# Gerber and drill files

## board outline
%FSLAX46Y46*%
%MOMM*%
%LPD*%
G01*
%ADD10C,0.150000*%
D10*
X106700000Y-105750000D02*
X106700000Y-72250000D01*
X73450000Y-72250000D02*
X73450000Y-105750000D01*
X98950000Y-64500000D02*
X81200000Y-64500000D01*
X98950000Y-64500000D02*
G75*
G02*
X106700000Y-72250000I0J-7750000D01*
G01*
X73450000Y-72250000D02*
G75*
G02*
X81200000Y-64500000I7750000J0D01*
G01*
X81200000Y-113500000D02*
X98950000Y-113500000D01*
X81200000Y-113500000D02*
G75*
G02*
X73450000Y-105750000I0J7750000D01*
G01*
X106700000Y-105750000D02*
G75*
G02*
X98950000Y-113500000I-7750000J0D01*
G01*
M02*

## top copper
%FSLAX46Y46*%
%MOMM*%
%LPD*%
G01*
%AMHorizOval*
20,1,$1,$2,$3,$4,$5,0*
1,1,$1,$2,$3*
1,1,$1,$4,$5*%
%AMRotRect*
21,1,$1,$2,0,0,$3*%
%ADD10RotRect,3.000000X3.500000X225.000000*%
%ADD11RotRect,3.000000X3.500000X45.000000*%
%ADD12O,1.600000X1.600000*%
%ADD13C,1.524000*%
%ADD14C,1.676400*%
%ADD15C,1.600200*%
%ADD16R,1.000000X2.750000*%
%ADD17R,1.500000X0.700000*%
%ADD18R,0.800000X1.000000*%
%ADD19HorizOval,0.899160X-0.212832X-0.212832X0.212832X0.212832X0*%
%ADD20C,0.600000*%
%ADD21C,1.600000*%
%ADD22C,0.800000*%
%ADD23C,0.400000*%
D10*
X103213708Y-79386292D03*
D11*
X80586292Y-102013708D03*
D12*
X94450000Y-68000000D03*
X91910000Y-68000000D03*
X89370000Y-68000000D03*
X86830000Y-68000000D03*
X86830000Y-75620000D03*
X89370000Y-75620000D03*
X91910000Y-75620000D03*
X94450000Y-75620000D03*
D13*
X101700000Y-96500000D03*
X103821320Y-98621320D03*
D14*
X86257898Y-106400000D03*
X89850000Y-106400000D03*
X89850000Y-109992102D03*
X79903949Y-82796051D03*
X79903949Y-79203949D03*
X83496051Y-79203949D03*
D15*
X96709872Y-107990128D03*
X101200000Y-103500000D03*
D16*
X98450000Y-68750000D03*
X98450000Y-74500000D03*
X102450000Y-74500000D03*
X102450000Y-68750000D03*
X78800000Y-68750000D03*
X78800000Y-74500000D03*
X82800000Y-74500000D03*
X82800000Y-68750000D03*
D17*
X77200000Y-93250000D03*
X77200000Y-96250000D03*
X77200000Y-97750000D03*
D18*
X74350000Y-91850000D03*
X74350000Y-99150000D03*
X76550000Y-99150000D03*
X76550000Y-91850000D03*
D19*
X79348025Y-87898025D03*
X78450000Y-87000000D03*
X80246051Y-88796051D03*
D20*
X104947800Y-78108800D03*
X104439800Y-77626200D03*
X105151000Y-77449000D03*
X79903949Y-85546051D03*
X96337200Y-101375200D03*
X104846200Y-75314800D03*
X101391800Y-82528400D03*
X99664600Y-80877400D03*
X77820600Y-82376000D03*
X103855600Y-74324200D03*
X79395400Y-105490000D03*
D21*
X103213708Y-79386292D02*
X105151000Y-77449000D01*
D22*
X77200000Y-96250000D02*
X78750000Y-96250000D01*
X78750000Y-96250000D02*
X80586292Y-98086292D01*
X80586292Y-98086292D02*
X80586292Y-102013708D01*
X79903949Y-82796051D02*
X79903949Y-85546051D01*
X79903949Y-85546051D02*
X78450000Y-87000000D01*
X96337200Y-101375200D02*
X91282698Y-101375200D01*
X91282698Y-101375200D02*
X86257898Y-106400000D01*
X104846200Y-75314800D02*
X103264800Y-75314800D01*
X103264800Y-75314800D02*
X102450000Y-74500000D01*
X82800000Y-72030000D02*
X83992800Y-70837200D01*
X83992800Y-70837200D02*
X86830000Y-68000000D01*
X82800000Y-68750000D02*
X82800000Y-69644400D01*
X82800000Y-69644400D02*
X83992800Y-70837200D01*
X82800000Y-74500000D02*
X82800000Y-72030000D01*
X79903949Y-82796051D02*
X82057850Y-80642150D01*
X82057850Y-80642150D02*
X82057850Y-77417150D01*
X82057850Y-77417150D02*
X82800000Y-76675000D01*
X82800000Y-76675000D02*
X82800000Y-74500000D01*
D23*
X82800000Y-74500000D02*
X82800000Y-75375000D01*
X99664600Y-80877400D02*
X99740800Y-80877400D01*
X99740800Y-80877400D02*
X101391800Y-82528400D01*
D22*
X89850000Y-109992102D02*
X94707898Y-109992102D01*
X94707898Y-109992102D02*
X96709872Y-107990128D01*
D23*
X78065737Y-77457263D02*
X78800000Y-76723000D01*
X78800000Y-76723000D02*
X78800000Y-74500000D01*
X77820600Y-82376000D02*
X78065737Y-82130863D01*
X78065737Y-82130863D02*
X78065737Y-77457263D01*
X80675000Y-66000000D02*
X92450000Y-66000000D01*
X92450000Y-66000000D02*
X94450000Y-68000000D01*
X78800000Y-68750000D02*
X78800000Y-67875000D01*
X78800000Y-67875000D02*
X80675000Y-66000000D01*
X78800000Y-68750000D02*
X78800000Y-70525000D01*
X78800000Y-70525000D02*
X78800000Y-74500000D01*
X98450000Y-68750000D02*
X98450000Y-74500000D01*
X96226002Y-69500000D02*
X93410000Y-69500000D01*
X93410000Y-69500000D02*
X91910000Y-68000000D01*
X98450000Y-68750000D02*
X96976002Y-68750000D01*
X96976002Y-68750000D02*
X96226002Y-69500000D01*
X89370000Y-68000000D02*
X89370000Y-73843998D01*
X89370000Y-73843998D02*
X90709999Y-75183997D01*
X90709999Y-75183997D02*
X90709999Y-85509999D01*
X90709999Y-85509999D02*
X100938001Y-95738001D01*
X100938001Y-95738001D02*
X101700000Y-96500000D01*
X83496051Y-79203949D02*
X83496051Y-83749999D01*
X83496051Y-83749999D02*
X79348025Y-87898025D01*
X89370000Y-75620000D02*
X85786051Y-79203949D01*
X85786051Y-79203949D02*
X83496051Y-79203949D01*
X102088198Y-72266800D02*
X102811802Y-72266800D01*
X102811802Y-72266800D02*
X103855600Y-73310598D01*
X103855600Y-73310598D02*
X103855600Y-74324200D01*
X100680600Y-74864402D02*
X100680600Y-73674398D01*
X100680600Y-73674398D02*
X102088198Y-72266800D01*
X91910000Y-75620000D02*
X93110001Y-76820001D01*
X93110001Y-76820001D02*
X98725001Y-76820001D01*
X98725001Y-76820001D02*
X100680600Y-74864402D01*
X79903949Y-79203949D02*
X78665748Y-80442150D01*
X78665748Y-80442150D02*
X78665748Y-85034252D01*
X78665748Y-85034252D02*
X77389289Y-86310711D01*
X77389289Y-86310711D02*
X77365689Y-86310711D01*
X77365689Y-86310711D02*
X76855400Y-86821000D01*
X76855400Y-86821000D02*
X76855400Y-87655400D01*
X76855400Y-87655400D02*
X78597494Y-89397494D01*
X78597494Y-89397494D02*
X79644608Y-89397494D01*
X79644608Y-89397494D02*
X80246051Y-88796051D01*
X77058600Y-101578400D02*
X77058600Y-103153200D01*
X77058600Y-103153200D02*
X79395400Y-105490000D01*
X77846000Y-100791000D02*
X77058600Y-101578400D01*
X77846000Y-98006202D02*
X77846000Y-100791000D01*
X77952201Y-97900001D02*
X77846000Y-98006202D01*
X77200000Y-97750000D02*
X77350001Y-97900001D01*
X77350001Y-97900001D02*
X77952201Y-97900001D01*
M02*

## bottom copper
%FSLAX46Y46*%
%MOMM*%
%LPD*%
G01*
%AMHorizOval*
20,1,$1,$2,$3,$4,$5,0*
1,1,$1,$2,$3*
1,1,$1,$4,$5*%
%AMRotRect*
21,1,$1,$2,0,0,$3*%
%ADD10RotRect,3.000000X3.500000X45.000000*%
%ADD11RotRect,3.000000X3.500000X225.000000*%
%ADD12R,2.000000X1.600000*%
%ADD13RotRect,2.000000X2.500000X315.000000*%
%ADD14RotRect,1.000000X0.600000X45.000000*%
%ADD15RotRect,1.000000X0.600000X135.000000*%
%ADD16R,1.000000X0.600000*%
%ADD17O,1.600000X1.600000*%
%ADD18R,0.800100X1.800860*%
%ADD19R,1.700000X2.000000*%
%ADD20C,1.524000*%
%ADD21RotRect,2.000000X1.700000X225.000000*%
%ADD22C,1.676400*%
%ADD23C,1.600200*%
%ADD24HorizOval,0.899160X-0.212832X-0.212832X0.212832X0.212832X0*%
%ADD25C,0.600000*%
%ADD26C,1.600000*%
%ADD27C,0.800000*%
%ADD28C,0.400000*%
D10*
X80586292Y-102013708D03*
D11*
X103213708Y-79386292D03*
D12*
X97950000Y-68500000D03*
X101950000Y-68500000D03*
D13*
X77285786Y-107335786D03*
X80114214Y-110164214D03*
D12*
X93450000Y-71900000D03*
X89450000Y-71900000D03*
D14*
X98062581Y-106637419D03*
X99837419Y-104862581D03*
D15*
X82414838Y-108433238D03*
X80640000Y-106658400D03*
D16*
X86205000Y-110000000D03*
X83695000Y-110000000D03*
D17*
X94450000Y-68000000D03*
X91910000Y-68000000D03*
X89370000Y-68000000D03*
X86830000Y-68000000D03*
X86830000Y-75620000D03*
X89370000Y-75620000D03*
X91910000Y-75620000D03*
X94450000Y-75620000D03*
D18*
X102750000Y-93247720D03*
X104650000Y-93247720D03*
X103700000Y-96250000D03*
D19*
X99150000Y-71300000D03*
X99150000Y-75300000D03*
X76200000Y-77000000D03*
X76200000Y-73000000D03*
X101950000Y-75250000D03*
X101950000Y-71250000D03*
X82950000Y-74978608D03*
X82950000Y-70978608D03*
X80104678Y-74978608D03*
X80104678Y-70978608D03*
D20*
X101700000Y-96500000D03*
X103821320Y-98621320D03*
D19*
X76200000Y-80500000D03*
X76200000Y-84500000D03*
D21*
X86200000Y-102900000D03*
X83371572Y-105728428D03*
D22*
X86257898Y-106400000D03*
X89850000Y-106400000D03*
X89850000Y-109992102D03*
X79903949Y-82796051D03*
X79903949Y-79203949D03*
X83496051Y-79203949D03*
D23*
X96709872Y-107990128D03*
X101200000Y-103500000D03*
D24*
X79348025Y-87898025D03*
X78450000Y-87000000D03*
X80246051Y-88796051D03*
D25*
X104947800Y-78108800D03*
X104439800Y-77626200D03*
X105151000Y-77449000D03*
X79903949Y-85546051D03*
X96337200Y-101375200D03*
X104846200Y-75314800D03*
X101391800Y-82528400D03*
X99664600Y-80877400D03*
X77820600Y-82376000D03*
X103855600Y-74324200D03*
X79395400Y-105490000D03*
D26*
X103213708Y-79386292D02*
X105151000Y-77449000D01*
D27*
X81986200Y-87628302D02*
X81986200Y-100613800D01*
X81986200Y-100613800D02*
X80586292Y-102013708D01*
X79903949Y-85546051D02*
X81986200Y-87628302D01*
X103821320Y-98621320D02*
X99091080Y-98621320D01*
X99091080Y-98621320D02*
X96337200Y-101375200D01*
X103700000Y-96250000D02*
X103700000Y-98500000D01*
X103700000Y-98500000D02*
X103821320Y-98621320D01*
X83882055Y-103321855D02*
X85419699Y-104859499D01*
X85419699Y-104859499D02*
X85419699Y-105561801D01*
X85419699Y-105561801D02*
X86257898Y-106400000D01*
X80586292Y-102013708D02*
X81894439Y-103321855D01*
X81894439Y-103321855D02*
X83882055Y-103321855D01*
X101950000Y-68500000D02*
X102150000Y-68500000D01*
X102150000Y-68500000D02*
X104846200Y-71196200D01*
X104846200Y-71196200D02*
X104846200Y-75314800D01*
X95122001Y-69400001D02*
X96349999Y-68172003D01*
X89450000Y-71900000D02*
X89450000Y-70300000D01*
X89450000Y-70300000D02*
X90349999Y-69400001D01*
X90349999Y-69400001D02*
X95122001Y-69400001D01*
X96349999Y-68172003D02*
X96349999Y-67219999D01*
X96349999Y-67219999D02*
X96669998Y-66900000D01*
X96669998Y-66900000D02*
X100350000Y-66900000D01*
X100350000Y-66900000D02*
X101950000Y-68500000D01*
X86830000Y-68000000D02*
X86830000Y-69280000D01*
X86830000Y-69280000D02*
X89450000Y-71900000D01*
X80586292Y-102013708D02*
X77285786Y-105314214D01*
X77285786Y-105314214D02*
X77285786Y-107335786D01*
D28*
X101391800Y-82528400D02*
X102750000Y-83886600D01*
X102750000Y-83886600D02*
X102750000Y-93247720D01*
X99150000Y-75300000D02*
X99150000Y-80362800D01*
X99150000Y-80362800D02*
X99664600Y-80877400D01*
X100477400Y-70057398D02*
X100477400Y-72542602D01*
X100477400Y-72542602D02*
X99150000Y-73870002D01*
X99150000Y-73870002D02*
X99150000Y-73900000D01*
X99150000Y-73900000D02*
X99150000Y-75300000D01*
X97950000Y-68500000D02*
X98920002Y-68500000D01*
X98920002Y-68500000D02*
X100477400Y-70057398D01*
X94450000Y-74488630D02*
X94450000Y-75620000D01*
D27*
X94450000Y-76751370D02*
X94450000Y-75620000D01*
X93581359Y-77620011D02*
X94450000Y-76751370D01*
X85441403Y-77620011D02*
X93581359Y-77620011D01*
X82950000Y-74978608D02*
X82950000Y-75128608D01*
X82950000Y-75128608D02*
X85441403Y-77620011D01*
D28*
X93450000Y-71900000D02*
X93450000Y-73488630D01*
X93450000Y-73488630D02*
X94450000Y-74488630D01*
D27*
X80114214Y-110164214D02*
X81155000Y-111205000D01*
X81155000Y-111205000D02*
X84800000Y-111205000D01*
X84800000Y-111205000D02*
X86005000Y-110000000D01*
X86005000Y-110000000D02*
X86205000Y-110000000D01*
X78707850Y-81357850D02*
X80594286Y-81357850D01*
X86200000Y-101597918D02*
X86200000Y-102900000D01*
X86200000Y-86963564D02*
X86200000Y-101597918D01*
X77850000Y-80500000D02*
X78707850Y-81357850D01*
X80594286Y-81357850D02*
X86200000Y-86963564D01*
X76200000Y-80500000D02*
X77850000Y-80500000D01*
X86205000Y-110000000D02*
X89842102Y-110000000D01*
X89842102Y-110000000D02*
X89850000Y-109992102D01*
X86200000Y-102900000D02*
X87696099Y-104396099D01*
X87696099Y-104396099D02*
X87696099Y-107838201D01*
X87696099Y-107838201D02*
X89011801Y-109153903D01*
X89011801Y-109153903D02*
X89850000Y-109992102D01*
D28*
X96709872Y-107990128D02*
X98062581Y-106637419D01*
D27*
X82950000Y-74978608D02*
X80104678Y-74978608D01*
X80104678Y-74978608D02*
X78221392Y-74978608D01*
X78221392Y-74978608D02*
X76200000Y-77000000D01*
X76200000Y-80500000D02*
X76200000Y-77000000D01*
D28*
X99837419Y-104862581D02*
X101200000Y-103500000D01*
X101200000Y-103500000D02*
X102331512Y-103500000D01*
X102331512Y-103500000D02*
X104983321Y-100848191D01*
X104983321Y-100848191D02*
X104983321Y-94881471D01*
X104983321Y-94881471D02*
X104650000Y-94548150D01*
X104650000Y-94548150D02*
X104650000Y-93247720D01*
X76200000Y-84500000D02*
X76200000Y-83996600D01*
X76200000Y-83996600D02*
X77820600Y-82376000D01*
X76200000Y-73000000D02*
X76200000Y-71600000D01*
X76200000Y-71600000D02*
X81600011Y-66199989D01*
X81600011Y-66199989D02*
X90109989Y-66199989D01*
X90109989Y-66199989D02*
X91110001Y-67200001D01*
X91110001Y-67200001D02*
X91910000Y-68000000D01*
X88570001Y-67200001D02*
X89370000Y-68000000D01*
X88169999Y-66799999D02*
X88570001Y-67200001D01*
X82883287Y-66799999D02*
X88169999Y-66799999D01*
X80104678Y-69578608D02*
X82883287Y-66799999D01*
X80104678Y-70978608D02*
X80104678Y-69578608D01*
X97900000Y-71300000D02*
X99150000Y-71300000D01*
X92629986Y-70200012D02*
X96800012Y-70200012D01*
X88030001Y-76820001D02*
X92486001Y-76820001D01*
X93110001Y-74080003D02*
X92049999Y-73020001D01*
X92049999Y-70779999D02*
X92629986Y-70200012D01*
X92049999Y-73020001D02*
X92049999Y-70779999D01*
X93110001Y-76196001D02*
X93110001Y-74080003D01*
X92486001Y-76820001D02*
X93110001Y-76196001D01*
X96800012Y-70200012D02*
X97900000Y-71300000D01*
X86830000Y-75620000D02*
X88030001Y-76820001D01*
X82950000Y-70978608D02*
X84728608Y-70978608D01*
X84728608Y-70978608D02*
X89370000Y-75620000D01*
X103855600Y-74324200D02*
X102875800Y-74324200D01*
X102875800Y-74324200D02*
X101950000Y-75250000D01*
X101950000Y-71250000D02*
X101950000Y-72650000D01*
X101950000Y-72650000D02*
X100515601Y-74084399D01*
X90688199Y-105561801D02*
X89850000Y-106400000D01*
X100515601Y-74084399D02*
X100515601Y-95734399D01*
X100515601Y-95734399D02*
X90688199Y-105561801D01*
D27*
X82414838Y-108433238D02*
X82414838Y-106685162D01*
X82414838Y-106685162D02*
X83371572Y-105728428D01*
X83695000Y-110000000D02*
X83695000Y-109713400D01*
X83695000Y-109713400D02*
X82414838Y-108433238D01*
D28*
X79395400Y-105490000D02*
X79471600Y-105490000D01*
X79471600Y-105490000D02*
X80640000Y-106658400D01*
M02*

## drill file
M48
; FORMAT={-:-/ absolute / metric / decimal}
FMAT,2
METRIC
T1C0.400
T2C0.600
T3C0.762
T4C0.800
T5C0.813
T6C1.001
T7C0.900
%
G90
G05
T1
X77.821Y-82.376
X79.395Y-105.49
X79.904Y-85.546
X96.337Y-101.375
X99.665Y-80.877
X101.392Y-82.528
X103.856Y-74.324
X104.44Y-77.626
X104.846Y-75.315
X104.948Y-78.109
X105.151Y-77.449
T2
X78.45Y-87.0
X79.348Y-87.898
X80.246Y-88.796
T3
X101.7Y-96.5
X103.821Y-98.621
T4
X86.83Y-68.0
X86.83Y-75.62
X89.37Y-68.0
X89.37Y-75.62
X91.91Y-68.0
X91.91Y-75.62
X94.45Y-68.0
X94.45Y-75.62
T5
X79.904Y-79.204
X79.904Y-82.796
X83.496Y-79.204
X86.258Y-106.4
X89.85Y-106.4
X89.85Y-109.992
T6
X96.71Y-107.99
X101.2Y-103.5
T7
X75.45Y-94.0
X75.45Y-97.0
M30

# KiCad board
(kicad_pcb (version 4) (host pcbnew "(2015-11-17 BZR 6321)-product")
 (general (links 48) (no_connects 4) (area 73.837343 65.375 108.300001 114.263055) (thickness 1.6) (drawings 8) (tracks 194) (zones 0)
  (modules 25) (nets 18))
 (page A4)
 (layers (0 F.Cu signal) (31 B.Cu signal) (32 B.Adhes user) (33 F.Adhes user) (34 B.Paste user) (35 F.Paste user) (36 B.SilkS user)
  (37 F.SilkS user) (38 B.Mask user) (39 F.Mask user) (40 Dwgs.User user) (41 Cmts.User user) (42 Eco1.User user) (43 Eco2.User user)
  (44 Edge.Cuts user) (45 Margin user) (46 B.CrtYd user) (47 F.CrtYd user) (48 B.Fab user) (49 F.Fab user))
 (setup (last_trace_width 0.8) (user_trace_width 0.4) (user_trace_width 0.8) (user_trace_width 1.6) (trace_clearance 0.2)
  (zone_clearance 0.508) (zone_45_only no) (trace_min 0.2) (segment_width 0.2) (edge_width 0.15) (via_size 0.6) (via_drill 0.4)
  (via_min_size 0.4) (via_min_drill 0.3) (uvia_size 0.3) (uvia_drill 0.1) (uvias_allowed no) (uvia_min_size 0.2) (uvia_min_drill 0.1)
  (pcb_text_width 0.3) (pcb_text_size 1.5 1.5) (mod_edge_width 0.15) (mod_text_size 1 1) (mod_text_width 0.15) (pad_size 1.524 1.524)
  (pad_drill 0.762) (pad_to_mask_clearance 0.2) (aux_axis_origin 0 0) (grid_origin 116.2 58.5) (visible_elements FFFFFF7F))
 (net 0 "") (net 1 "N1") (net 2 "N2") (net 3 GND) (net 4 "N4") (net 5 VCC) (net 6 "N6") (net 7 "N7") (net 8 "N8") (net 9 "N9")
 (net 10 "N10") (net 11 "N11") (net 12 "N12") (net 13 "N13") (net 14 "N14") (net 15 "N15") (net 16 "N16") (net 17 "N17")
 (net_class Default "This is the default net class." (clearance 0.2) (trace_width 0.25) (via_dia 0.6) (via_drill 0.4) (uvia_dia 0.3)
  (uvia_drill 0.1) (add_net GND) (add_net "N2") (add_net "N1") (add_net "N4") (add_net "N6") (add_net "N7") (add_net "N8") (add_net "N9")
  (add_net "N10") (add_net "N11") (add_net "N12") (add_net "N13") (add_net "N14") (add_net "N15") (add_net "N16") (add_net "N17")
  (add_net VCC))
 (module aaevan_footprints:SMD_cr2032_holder (layer F.Cu) (at 91.9 90.7 225)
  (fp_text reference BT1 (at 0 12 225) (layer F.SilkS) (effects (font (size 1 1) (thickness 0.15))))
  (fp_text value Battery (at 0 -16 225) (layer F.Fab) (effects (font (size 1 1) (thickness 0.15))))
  (pad 2 smd rect (at -16 0 225) (size 3 3.5) (layers F.Cu F.Paste F.Mask) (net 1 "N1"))
  (pad 1 smd rect (at 16 0 45) (size 3 3.5) (layers F.Cu F.Paste F.Mask) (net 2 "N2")))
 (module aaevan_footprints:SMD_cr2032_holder (layer B.Cu) (at 91.9 90.7 45)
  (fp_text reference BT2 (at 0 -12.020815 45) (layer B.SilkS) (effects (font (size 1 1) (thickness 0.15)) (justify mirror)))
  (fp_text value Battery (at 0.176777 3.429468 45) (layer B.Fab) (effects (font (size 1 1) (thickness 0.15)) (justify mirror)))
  (pad 2 smd rect (at -16 0 45) (size 3 3.5) (layers B.Cu B.Paste B.Mask) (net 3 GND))
  (pad 1 smd rect (at 16 0 225) (size 3 3.5) (layers B.Cu B.Paste B.Mask) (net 1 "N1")))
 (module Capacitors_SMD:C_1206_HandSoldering (layer B.Cu) (at 99.95 68.5)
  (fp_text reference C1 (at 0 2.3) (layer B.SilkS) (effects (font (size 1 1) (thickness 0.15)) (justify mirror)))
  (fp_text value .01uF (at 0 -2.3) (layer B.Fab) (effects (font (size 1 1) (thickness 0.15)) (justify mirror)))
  (pad 1 smd rect (at -2 0) (size 2 1.6) (layers B.Cu B.Paste B.Mask) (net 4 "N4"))
  (pad 2 smd rect (at 2 0) (size 2 1.6) (layers B.Cu B.Paste B.Mask) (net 3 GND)))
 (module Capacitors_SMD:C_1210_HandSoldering (layer B.Cu) (at 78.7 108.75 315)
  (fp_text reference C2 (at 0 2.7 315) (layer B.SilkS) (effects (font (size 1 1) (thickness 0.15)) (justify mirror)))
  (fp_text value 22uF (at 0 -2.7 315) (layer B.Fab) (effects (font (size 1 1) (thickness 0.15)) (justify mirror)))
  (pad 1 smd rect (at -2 0 315) (size 2 2.5) (layers B.Cu B.Paste B.Mask) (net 3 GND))
  (pad 2 smd rect (at 2 0 315) (size 2 2.5) (layers B.Cu B.Paste B.Mask) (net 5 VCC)))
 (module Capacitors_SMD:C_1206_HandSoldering (layer B.Cu) (at 91.45 71.9 180)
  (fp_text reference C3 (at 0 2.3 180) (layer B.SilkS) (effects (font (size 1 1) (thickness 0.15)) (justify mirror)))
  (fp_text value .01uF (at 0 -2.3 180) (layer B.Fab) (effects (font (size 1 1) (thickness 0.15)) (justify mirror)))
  (pad 1 smd rect (at -2 0 180) (size 2 1.6) (layers B.Cu B.Paste B.Mask) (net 5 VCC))
  (pad 2 smd rect (at 2 0 180) (size 2 1.6) (layers B.Cu B.Paste B.Mask) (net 3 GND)))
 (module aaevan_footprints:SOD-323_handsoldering (layer B.Cu) (at 98.95 105.75 45)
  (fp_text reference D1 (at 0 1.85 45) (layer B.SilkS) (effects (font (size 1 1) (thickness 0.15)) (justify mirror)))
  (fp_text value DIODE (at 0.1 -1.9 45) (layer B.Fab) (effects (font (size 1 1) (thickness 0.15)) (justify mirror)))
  (pad 1 smd rect (at -1.255 0 45) (size 1 0.6) (layers B.Cu B.Paste B.Mask) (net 5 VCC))
  (pad 2 smd rect (at 1.255 0 45) (size 1 0.6) (layers B.Cu B.Paste B.Mask) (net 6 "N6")))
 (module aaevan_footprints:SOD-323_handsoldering (layer B.Cu) (at 81.527419 107.545819 135)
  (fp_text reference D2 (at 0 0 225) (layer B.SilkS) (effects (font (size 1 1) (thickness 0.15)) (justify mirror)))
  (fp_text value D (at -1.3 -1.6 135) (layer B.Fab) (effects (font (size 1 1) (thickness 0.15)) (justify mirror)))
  (pad 1 smd rect (at -1.255 0 135) (size 1 0.6) (layers B.Cu B.Paste B.Mask) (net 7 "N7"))
  (pad 2 smd rect (at 1.255 0 135) (size 1 0.6) (layers B.Cu B.Paste B.Mask) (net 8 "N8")))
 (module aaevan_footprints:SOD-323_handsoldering (layer B.Cu) (at 84.95 110 180)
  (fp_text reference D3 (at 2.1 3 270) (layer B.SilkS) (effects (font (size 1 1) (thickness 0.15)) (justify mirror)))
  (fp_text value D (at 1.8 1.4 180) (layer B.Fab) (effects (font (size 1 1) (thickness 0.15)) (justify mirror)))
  (pad 1 smd rect (at -1.255 0 180) (size 1 0.6) (layers B.Cu B.Paste B.Mask) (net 5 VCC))
  (pad 2 smd rect (at 1.255 0 180) (size 1 0.6) (layers B.Cu B.Paste B.Mask) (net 7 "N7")))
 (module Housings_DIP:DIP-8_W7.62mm (layer F.Cu) (at 94.45 68 270)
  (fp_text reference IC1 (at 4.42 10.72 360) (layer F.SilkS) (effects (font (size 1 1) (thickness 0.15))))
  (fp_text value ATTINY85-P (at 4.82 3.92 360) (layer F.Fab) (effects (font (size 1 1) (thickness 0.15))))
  (pad 1 thru_hole oval (at 0 0 270) (size 1.6 1.6) (drill 0.8) (layers *.Cu *.Mask F.SilkS) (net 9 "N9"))
  (pad 2 thru_hole oval (at 0 2.54 270) (size 1.6 1.6) (drill 0.8) (layers *.Cu *.Mask F.SilkS) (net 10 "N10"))
  (pad 3 thru_hole oval (at 0 5.08 270) (size 1.6 1.6) (drill 0.8) (layers *.Cu *.Mask F.SilkS) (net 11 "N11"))
  (pad 4 thru_hole oval (at 0 7.62 270) (size 1.6 1.6) (drill 0.8) (layers *.Cu *.Mask F.SilkS) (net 3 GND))
  (pad 5 thru_hole oval (at 7.62 7.62 270) (size 1.6 1.6) (drill 0.8) (layers *.Cu *.Mask F.SilkS) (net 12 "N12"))
  (pad 6 thru_hole oval (at 7.62 5.08 270) (size 1.6 1.6) (drill 0.8) (layers *.Cu *.Mask F.SilkS) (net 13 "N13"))
  (pad 7 thru_hole oval (at 7.62 2.54 270) (size 1.6 1.6) (drill 0.8) (layers *.Cu *.Mask F.SilkS) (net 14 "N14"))
  (pad 8 thru_hole oval (at 7.62 0 270) (size 1.6 1.6) (drill 0.8) (layers *.Cu *.Mask F.SilkS) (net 5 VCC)))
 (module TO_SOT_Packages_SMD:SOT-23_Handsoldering (layer B.Cu) (at 103.7 94.74886)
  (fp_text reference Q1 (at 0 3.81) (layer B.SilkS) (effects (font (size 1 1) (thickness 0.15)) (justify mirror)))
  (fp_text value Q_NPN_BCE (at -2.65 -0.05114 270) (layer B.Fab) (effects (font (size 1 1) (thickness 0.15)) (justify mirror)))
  (pad 1 smd rect (at -0.95 -1.50114) (size 0.8001 1.80086) (layers B.Cu B.Paste B.Mask) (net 4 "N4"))
  (pad 2 smd rect (at 0.95 -1.50114) (size 0.8001 1.80086) (layers B.Cu B.Paste B.Mask) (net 6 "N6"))
  (pad 3 smd rect (at 0 1.50114) (size 0.8001 1.80086) (layers B.Cu B.Paste B.Mask) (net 3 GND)))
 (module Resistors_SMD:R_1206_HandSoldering (layer B.Cu) (at 99.15 73.3 270)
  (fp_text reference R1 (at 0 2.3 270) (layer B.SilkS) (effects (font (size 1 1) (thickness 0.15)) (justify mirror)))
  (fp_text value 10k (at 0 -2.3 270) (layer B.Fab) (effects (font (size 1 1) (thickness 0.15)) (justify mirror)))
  (pad 1 smd rect (at -2 0 270) (size 2 1.7) (layers B.Cu B.Paste B.Mask) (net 12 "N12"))
  (pad 2 smd rect (at 2 0 270) (size 2 1.7) (layers B.Cu B.Paste B.Mask) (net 4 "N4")))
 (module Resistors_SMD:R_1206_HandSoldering (layer B.Cu) (at 76.2 75 90)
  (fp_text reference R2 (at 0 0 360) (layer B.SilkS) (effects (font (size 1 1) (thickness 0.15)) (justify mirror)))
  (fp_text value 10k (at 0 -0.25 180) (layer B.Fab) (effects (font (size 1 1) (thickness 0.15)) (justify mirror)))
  (pad 1 smd rect (at -2 0 90) (size 2 1.7) (layers B.Cu B.Paste B.Mask) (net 5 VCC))
  (pad 2 smd rect (at 2 0 90) (size 2 1.7) (layers B.Cu B.Paste B.Mask) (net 10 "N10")))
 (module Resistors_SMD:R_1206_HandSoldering (layer B.Cu) (at 101.95 73.25 90)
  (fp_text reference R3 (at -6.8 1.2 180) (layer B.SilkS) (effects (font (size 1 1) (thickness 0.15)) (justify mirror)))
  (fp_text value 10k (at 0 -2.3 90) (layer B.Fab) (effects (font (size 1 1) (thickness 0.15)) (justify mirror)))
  (pad 1 smd rect (at -2 0 90) (size 2 1.7) (layers B.Cu B.Paste B.Mask) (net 14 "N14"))
  (pad 2 smd rect (at 2 0 90) (size 2 1.7) (layers B.Cu B.Paste B.Mask) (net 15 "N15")))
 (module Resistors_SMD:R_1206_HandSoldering (layer B.Cu) (at 82.95 72.978608 90)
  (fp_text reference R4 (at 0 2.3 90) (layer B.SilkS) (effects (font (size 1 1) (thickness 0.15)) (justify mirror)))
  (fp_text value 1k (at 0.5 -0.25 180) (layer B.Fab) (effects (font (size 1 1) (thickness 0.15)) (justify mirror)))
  (pad 1 smd rect (at -2 0 90) (size 2 1.7) (layers B.Cu B.Paste B.Mask) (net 5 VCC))
  (pad 2 smd rect (at 2 0 90) (size 2 1.7) (layers B.Cu B.Paste B.Mask) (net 13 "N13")))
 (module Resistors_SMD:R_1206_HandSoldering (layer B.Cu) (at 80.104678 72.978608 90)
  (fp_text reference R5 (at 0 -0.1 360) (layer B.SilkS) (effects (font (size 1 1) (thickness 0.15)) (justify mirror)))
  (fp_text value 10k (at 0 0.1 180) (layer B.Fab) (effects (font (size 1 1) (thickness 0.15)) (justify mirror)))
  (pad 1 smd rect (at -2 0 90) (size 2 1.7) (layers B.Cu B.Paste B.Mask) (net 5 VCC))
  (pad 2 smd rect (at 2 0 90) (size 2 1.7) (layers B.Cu B.Paste B.Mask) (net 11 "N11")))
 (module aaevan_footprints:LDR (layer F.Cu) (at 102.76066 97.56066 315)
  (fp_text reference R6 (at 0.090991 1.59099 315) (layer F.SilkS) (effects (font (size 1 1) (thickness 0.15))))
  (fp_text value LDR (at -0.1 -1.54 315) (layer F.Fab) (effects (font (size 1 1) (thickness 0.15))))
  (pad 1 thru_hole circle (at -1.5 0 315) (size 1.524 1.524) (drill 0.762) (layers *.Cu *.Mask F.SilkS) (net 11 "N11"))
  (pad 2 thru_hole circle (at 1.5 0 315) (size 1.524 1.524) (drill 0.762) (layers *.Cu *.Mask F.SilkS) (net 3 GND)))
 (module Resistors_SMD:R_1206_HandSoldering (layer B.Cu) (at 76.2 82.5 270)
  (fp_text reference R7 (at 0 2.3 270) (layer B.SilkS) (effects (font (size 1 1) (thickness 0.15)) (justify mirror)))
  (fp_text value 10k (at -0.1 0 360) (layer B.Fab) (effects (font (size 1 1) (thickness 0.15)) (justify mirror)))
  (pad 1 smd rect (at -2 0 270) (size 2 1.7) (layers B.Cu B.Paste B.Mask) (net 5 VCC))
  (pad 2 smd rect (at 2 0 270) (size 2 1.7) (layers B.Cu B.Paste B.Mask) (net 9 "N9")))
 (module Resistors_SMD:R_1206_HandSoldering (layer B.Cu) (at 84.785786 104.314214 225)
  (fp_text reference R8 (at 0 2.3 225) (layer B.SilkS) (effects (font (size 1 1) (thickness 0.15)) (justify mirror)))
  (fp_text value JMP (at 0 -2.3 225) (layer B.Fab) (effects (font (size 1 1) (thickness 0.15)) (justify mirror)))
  (pad 1 smd rect (at -2 0 225) (size 2 1.7) (layers B.Cu B.Paste B.Mask) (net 5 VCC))
  (pad 2 smd rect (at 2 0 225) (size 2 1.7) (layers B.Cu B.Paste B.Mask) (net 7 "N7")))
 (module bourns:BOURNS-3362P (layer F.Cu) (at 88.053949 108.196051 315)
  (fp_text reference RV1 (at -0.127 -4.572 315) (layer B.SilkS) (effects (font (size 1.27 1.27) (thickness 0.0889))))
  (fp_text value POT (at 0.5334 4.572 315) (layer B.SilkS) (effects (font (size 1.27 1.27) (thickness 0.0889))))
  (pad 1 thru_hole circle (at -2.54 0 315) (size 1.6764 3.3528) (drill 0.8128) (layers *.Cu F.Paste F.SilkS F.Mask) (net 3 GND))
  (pad 2 thru_hole circle (at 0 -2.54 315) (size 1.6764 3.3528) (drill 0.8128) (layers *.Cu F.Paste F.SilkS F.Mask) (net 15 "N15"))
  (pad 3 thru_hole circle (at 2.54 0 315) (size 1.6764 3.3528) (drill 0.8128) (layers *.Cu F.Paste F.SilkS F.Mask) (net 5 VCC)))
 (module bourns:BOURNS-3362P (layer F.Cu) (at 81.7 81 45)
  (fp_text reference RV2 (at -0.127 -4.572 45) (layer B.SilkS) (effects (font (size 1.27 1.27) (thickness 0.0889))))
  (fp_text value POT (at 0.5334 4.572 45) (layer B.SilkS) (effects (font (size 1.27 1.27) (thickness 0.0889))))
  (pad 1 thru_hole circle (at -2.54 0 45) (size 1.6764 3.3528) (drill 0.8128) (layers *.Cu F.Paste F.SilkS F.Mask) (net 3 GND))
  (pad 2 thru_hole circle (at 0 -2.54 45) (size 1.6764 3.3528) (drill 0.8128) (layers *.Cu F.Paste F.SilkS F.Mask) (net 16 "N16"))
  (pad 3 thru_hole circle (at 2.54 0 45) (size 1.6764 3.3528) (drill 0.8128) (layers *.Cu F.Paste F.SilkS F.Mask) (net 13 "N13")))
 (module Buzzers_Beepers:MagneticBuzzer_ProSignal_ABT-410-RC (layer F.Cu) (at 96.709872 107.990128 45)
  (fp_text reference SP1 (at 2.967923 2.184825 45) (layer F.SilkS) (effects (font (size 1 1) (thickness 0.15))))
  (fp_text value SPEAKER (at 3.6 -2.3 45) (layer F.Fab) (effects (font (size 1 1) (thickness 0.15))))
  (pad 1 thru_hole circle (at 0 0 45) (size 1.6002 1.6002) (drill 1.00076) (layers *.Cu *.Mask F.SilkS) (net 5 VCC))
  (pad 2 thru_hole circle (at 6.35 0 45) (size 1.6002 1.6002) (drill 1.00076) (layers *.Cu *.Mask F.SilkS) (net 6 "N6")))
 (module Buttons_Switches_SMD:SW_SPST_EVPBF (layer F.Cu) (at 100.45 71.625 90)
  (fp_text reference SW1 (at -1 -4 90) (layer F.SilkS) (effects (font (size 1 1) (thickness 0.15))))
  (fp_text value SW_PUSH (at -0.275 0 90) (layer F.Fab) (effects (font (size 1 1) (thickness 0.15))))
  (pad 1 smd rect (at 2.875 -2 90) (size 2.75 1) (layers F.Cu F.Paste F.Mask) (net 10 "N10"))
  (pad 1 smd rect (at -2.875 -2 90) (size 2.75 1) (layers F.Cu F.Paste F.Mask) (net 10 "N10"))
  (pad 2 smd rect (at -2.875 2 90) (size 2.75 1) (layers F.Cu F.Paste F.Mask) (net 3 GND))
  (pad 2 smd rect (at 2.875 2 90) (size 2.75 1) (layers F.Cu F.Paste F.Mask) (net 3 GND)))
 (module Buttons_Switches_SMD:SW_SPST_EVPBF (layer F.Cu) (at 80.8 71.625 90)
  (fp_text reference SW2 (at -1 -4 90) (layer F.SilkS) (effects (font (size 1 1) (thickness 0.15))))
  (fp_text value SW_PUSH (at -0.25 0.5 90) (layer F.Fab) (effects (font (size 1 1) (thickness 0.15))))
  (pad 1 smd rect (at 2.875 -2 90) (size 2.75 1) (layers F.Cu F.Paste F.Mask) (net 9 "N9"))
  (pad 1 smd rect (at -2.875 -2 90) (size 2.75 1) (layers F.Cu F.Paste F.Mask) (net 9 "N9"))
  (pad 2 smd rect (at -2.875 2 90) (size 2.75 1) (layers F.Cu F.Paste F.Mask) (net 3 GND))
  (pad 2 smd rect (at 2.875 2 90) (size 2.75 1) (layers F.Cu F.Paste F.Mask) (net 3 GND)))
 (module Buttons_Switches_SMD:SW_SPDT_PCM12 (layer F.Cu) (at 75.775 95.5 270)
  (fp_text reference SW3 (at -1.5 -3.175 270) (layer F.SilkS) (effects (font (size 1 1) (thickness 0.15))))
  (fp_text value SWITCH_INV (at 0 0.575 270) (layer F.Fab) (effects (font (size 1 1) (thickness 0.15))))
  (pad "" np_thru_hole circle (at -1.5 0.325 270) (size 0.9 0.9) (drill 0.9) (layers *.Cu *.Mask))
  (pad "" np_thru_hole circle (at 1.5 0.325 270) (size 0.9 0.9) (drill 0.9) (layers *.Cu *.Mask))
  (pad 1 smd rect (at -2.25 -1.425 270) (size 0.7 1.5) (layers F.Cu F.Paste F.Mask) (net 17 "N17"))
  (pad 2 smd rect (at 0.75 -1.425 270) (size 0.7 1.5) (layers F.Cu F.Paste F.Mask) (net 2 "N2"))
  (pad 3 smd rect (at 2.25 -1.425 270) (size 0.7 1.5) (layers F.Cu F.Paste F.Mask) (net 8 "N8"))
  (pad "" smd rect (at -3.65 1.425 270) (size 1 0.8) (layers F.Cu F.Paste F.Mask))
  (pad "" smd rect (at 3.65 1.425 270) (size 1 0.8) (layers F.Cu F.Paste F.Mask))
  (pad "" smd rect (at 3.65 -0.775 270) (size 1 0.8) (layers F.Cu F.Paste F.Mask))
  (pad "" smd rect (at -3.65 -0.775 270) (size 1 0.8) (layers F.Cu F.Paste F.Mask)))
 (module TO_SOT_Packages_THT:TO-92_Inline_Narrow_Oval (layer F.Cu) (at 80.246051 88.796051 135)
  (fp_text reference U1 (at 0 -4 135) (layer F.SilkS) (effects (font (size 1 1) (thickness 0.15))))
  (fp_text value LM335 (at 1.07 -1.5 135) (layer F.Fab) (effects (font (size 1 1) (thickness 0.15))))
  (pad 2 thru_hole oval (at 1.27 0 315) (size 0.89916 1.50114) (drill 0.6) (layers *.Cu *.Mask F.SilkS) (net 13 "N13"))
  (pad 3 thru_hole oval (at 2.54 0 315) (size 0.89916 1.50114) (drill 0.6) (layers *.Cu *.Mask F.SilkS) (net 3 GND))
  (pad 1 thru_hole oval (at 0 0 315) (size 0.89916 1.50114) (drill 0.6) (layers *.Cu *.Mask F.SilkS) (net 16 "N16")))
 (gr_line (start 106.7 105.75) (end 106.7 72.25) (layer Edge.Cuts) (width 0.15))
 (gr_line (start 73.45 72.25) (end 73.45 105.75) (layer Edge.Cuts) (width 0.15))
 (gr_line (start 98.95 64.5) (end 81.2 64.5) (layer Edge.Cuts) (width 0.15))
 (gr_arc (start 98.95 72.25) (end 98.95 64.5) (angle 90) (layer Edge.Cuts) (width 0.15))
 (gr_arc (start 81.2 72.25) (end 73.45 72.25) (angle 90) (layer Edge.Cuts) (width 0.15))
 (gr_line (start 81.2 113.5) (end 98.95 113.5) (layer Edge.Cuts) (width 0.15))
 (gr_arc (start 81.2 105.75) (end 81.2 113.5) (angle 90) (layer Edge.Cuts) (width 0.15))
 (gr_arc (start 98.95 105.75) (end 106.7 105.75) (angle 90) (layer Edge.Cuts) (width 0.15))
 (via (at 104.9478 78.1088) (size 0.6) (drill 0.4) (layers F.Cu B.Cu) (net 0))
 (via (at 104.4398 77.6262) (size 0.6) (drill 0.4) (layers F.Cu B.Cu) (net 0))
 (segment (start 81.2 68.75) (end 79.7 68.75) (width 0.25) (layer Dwgs.User) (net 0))
 (segment (start 103.213708 79.386292) (end 105.151 77.449) (width 1.6) (layer F.Cu) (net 1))
 (via (at 105.151 77.449) (size 0.6) (drill 0.4) (layers F.Cu B.Cu) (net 1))
 (segment (start 103.213708 79.386292) (end 105.151 77.449) (width 1.6) (layer B.Cu) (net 1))
 (segment (start 77.2 96.25) (end 78.75 96.25) (width 0.8) (layer F.Cu) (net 2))
 (segment (start 78.75 96.25) (end 80.586292 98.086292) (width 0.8) (layer F.Cu) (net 2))
 (segment (start 80.586292 98.086292) (end 80.586292 102.013708) (width 0.8) (layer F.Cu) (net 2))
 (segment (start 81.9862 87.628302) (end 81.9862 100.6138) (width 0.8) (layer B.Cu) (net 3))
 (segment (start 81.9862 100.6138) (end 80.586292 102.013708) (width 0.8) (layer B.Cu) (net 3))
 (segment (start 79.903949 85.546051) (end 81.9862 87.628302) (width 0.8) (layer B.Cu) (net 3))
 (via (at 79.903949 85.546051) (size 0.6) (drill 0.4) (layers F.Cu B.Cu) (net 3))
 (segment (start 79.903949 82.796051) (end 79.903949 85.546051) (width 0.8) (layer F.Cu) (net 3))
 (segment (start 79.903949 85.546051) (end 78.45 87) (width 0.8) (layer F.Cu) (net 3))
 (segment (start 96.3372 101.3752) (end 91.282698 101.3752) (width 0.8) (layer F.Cu) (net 3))
 (segment (start 91.282698 101.3752) (end 86.257898 106.4) (width 0.8) (layer F.Cu) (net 3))
 (segment (start 103.82132 98.62132) (end 99.09108 98.62132) (width 0.8) (layer B.Cu) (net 3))
 (segment (start 99.09108 98.62132) (end 96.3372 101.3752) (width 0.8) (layer B.Cu) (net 3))
 (via (at 96.3372 101.3752) (size 0.6) (drill 0.4) (layers F.Cu B.Cu) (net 3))
 (segment (start 103.7 96.25) (end 103.7 98.5) (width 0.8) (layer B.Cu) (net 3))
 (segment (start 103.7 98.5) (end 103.82132 98.62132) (width 0.8) (layer B.Cu) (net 3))
 (segment (start 83.882055 103.321855) (end 85.419699 104.859499) (width 0.8) (layer B.Cu) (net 3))
 (segment (start 85.419699 104.859499) (end 85.419699 105.561801) (width 0.8) (layer B.Cu) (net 3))
 (segment (start 85.419699 105.561801) (end 86.257898 106.4) (width 0.8) (layer B.Cu) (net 3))
 (segment (start 80.586292 102.013708) (end 81.894439 103.321855) (width 0.8) (layer B.Cu) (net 3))
 (segment (start 81.894439 103.321855) (end 83.882055 103.321855) (width 0.8) (layer B.Cu) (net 3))
 (segment (start 104.8462 75.3148) (end 103.2648 75.3148) (width 0.8) (layer F.Cu) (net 3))
 (segment (start 103.2648 75.3148) (end 102.45 74.5) (width 0.8) (layer F.Cu) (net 3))
 (segment (start 101.95 68.5) (end 102.15 68.5) (width 0.8) (layer B.Cu) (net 3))
 (segment (start 102.15 68.5) (end 104.8462 71.1962) (width 0.8) (layer B.Cu) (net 3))
 (segment (start 104.8462 71.1962) (end 104.8462 75.3148) (width 0.8) (layer B.Cu) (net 3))
 (via (at 104.8462 75.3148) (size 0.6) (drill 0.4) (layers F.Cu B.Cu) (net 3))
 (segment (start 95.122001 69.400001) (end 96.349999 68.172003) (width 0.8) (layer B.Cu) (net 3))
 (segment (start 89.45 71.9) (end 89.45 70.3) (width 0.8) (layer B.Cu) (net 3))
 (segment (start 89.45 70.3) (end 90.349999 69.400001) (width 0.8) (layer B.Cu) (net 3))
 (segment (start 90.349999 69.400001) (end 95.122001 69.400001) (width 0.8) (layer B.Cu) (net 3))
 (segment (start 96.349999 68.172003) (end 96.349999 67.219999) (width 0.8) (layer B.Cu) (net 3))
 (segment (start 96.349999 67.219999) (end 96.669998 66.9) (width 0.8) (layer B.Cu) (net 3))
 (segment (start 96.669998 66.9) (end 100.35 66.9) (width 0.8) (layer B.Cu) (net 3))
 (segment (start 100.35 66.9) (end 101.95 68.5) (width 0.8) (layer B.Cu) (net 3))
 (segment (start 86.83 68) (end 86.83 69.28) (width 0.8) (layer B.Cu) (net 3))
 (segment (start 86.83 69.28) (end 89.45 71.9) (width 0.8) (layer B.Cu) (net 3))
 (segment (start 82.8 72.03) (end 83.9928 70.8372) (width 0.8) (layer F.Cu) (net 3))
 (segment (start 83.9928 70.8372) (end 86.83 68) (width 0.8) (layer F.Cu) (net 3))
 (segment (start 82.8 68.75) (end 82.8 69.6444) (width 0.8) (layer F.Cu) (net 3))
 (segment (start 82.8 69.6444) (end 83.9928 70.8372) (width 0.8) (layer F.Cu) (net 3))
 (segment (start 82.8 74.5) (end 82.8 72.03) (width 0.8) (layer F.Cu) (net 3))
 (segment (start 79.903949 82.796051) (end 82.05785 80.64215) (width 0.8) (layer F.Cu) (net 3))
 (segment (start 82.05785 80.64215) (end 82.05785 77.41715) (width 0.8) (layer F.Cu) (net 3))
 (segment (start 82.05785 77.41715) (end 82.8 76.675) (width 0.8) (layer F.Cu) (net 3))
 (segment (start 82.8 76.675) (end 82.8 74.5) (width 0.8) (layer F.Cu) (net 3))
 (segment (start 80.586292 102.013708) (end 77.285786 105.314214) (width 0.8) (layer B.Cu) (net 3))
 (segment (start 77.285786 105.314214) (end 77.285786 107.335786) (width 0.8) (layer B.Cu) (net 3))
 (segment (start 82.8 74.5) (end 82.8 75.375) (width 0.4) (layer F.Cu) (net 3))
 (segment (start 101.3918 82.5284) (end 102.75 83.8866) (width 0.4) (layer B.Cu) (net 4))
 (segment (start 102.75 83.8866) (end 102.75 93.24772) (width 0.4) (layer B.Cu) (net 4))
 (segment (start 99.6646 80.8774) (end 99.7408 80.8774) (width 0.4) (layer F.Cu) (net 4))
 (segment (start 99.7408 80.8774) (end 101.3918 82.5284) (width 0.4) (layer F.Cu) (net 4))
 (via (at 101.3918 82.5284) (size 0.6) (drill 0.4) (layers F.Cu B.Cu) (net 4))
 (segment (start 99.15 75.3) (end 99.15 80.3628) (width 0.4) (layer B.Cu) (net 4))
 (segment (start 99.15 80.3628) (end 99.6646 80.8774) (width 0.4) (layer B.Cu) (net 4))
 (via (at 99.6646 80.8774) (size 0.6) (drill 0.4) (layers F.Cu B.Cu) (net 4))
 (segment (start 100.4774 70.057398) (end 100.4774 72.542602) (width 0.4) (layer B.Cu) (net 4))
 (segment (start 100.4774 72.542602) (end 99.15 73.870002) (width 0.4) (layer B.Cu) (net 4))
 (segment (start 99.15 73.870002) (end 99.15 73.9) (width 0.4) (layer B.Cu) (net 4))
 (segment (start 99.15 73.9) (end 99.15 75.3) (width 0.4) (layer B.Cu) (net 4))
 (segment (start 97.95 68.5) (end 98.920002 68.5) (width 0.4) (layer B.Cu) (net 4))
 (segment (start 98.920002 68.5) (end 100.4774 70.057398) (width 0.4) (layer B.Cu) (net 4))
 (segment (start 94.45 74.48863) (end 94.45 75.62) (width 0.4) (layer B.Cu) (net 5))
 (segment (start 94.45 76.75137) (end 94.45 75.62) (width 0.8) (layer B.Cu) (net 5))
 (segment (start 93.581359 77.620011) (end 94.45 76.75137) (width 0.8) (layer B.Cu) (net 5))
 (segment (start 85.441403 77.620011) (end 93.581359 77.620011) (width 0.8) (layer B.Cu) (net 5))
 (segment (start 82.95 74.978608) (end 82.95 75.128608) (width 0.8) (layer B.Cu) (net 5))
 (segment (start 82.95 75.128608) (end 85.441403 77.620011) (width 0.8) (layer B.Cu) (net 5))
 (segment (start 93.45 71.9) (end 93.45 73.48863) (width 0.4) (layer B.Cu) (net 5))
 (segment (start 93.45 73.48863) (end 94.45 74.48863) (width 0.4) (layer B.Cu) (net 5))
 (segment (start 80.114214 110.164214) (end 81.155 111.205) (width 0.8) (layer B.Cu) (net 5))
 (segment (start 81.155 111.205) (end 84.8 111.205) (width 0.8) (layer B.Cu) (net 5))
 (segment (start 84.8 111.205) (end 86.005 110) (width 0.8) (layer B.Cu) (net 5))
 (segment (start 86.005 110) (end 86.205 110) (width 0.8) (layer B.Cu) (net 5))
 (segment (start 78.70785 81.35785) (end 80.594286 81.35785) (width 0.8) (layer B.Cu) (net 5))
 (segment (start 86.2 101.597918) (end 86.2 102.9) (width 0.8) (layer B.Cu) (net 5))
 (segment (start 86.2 86.963564) (end 86.2 101.597918) (width 0.8) (layer B.Cu) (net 5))
 (segment (start 77.85 80.5) (end 78.70785 81.35785) (width 0.8) (layer B.Cu) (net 5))
 (segment (start 80.594286 81.35785) (end 86.2 86.963564) (width 0.8) (layer B.Cu) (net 5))
 (segment (start 76.2 80.5) (end 77.85 80.5) (width 0.8) (layer B.Cu) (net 5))
 (segment (start 89.85 109.992102) (end 94.707898 109.992102) (width 0.8) (layer F.Cu) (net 5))
 (segment (start 94.707898 109.992102) (end 96.709872 107.990128) (width 0.8) (layer F.Cu) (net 5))
 (segment (start 86.205 110) (end 89.842102 110) (width 0.8) (layer B.Cu) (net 5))
 (segment (start 89.842102 110) (end 89.85 109.992102) (width 0.8) (layer B.Cu) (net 5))
 (segment (start 86.2 102.9) (end 87.696099 104.396099) (width 0.8) (layer B.Cu) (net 5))
 (segment (start 87.696099 104.396099) (end 87.696099 107.838201) (width 0.8) (layer B.Cu) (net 5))
 (segment (start 87.696099 107.838201) (end 89.011801 109.153903) (width 0.8) (layer B.Cu) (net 5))
 (segment (start 89.011801 109.153903) (end 89.85 109.992102) (width 0.8) (layer B.Cu) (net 5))
 (segment (start 96.709872 107.990128) (end 98.062581 106.637419) (width 0.4) (layer B.Cu) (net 5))
 (segment (start 82.95 74.978608) (end 80.104678 74.978608) (width 0.8) (layer B.Cu) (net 5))
 (segment (start 80.104678 74.978608) (end 78.221392 74.978608) (width 0.8) (layer B.Cu) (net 5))
 (segment (start 78.221392 74.978608) (end 76.2 77) (width 0.8) (layer B.Cu) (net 5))
 (segment (start 76.2 80.5) (end 76.2 77) (width 0.8) (layer B.Cu) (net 5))
 (segment (start 99.837419 104.862581) (end 101.2 103.5) (width 0.4) (layer B.Cu) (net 6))
 (segment (start 101.2 103.5) (end 102.331512 103.5) (width 0.4) (layer B.Cu) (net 6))
 (segment (start 102.331512 103.5) (end 104.983321 100.848191) (width 0.4) (layer B.Cu) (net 6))
 (segment (start 104.983321 100.848191) (end 104.983321 94.881471) (width 0.4) (layer B.Cu) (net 6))
 (segment (start 104.983321 94.881471) (end 104.65 94.54815) (width 0.4) (layer B.Cu) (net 6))
 (segment (start 104.65 94.54815) (end 104.65 93.24772) (width 0.4) (layer B.Cu) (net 6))
 (segment (start 78.065737 77.457263) (end 78.8 76.723) (width 0.4) (layer F.Cu) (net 9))
 (segment (start 78.8 76.723) (end 78.8 74.5) (width 0.4) (layer F.Cu) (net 9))
 (segment (start 77.8206 82.376) (end 78.065737 82.130863) (width 0.4) (layer F.Cu) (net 9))
 (segment (start 78.065737 82.130863) (end 78.065737 77.457263) (width 0.4) (layer F.Cu) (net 9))
 (segment (start 76.2 84.5) (end 76.2 83.9966) (width 0.4) (layer B.Cu) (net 9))
 (segment (start 76.2 83.9966) (end 77.8206 82.376) (width 0.4) (layer B.Cu) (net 9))
 (via (at 77.8206 82.376) (size 0.6) (drill 0.4) (layers F.Cu B.Cu) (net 9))
 (segment (start 80.675 66) (end 92.45 66) (width 0.4) (layer F.Cu) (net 9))
 (segment (start 92.45 66) (end 94.45 68) (width 0.4) (layer F.Cu) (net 9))
 (segment (start 78.8 68.75) (end 78.8 67.875) (width 0.4) (layer F.Cu) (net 9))
 (segment (start 78.8 67.875) (end 80.675 66) (width 0.4) (layer F.Cu) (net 9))
 (segment (start 78.8 68.75) (end 78.8 70.525) (width 0.4) (layer F.Cu) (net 9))
 (segment (start 78.8 70.525) (end 78.8 74.5) (width 0.4) (layer F.Cu) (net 9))
 (segment (start 76.2 73) (end 76.2 71.6) (width 0.4) (layer B.Cu) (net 10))
 (segment (start 76.2 71.6) (end 81.600011 66.199989) (width 0.4) (layer B.Cu) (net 10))
 (segment (start 81.600011 66.199989) (end 90.109989 66.199989) (width 0.4) (layer B.Cu) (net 10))
 (segment (start 90.109989 66.199989) (end 91.110001 67.200001) (width 0.4) (layer B.Cu) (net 10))
 (segment (start 91.110001 67.200001) (end 91.91 68) (width 0.4) (layer B.Cu) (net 10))
 (segment (start 98.45 68.75) (end 98.45 74.5) (width 0.4) (layer F.Cu) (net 10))
 (segment (start 96.226002 69.5) (end 93.41 69.5) (width 0.4) (layer F.Cu) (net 10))
 (segment (start 93.41 69.5) (end 91.91 68) (width 0.4) (layer F.Cu) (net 10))
 (segment (start 98.45 68.75) (end 96.976002 68.75) (width 0.4) (layer F.Cu) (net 10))
 (segment (start 96.976002 68.75) (end 96.226002 69.5) (width 0.4) (layer F.Cu) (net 10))
 (segment (start 88.570001 67.200001) (end 89.37 68) (width 0.4) (layer B.Cu) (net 11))
 (segment (start 88.169999 66.799999) (end 88.570001 67.200001) (width 0.4) (layer B.Cu) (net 11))
 (segment (start 82.883287 66.799999) (end 88.169999 66.799999) (width 0.4) (layer B.Cu) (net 11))
 (segment (start 80.104678 69.578608) (end 82.883287 66.799999) (width 0.4) (layer B.Cu) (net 11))
 (segment (start 80.104678 70.978608) (end 80.104678 69.578608) (width 0.4) (layer B.Cu) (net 11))
 (segment (start 89.37 68) (end 89.37 73.843998) (width 0.4) (layer F.Cu) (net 11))
 (segment (start 89.37 73.843998) (end 90.709999 75.183997) (width 0.4) (layer F.Cu) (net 11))
 (segment (start 90.709999 75.183997) (end 90.709999 85.509999) (width 0.4) (layer F.Cu) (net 11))
 (segment (start 90.709999 85.509999) (end 100.938001 95.738001) (width 0.4) (layer F.Cu) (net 11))
 (segment (start 100.938001 95.738001) (end 101.7 96.5) (width 0.4) (layer F.Cu) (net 11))
 (segment (start 97.9 71.3) (end 99.15 71.3) (width 0.4) (layer B.Cu) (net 12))
 (segment (start 92.629986 70.200012) (end 96.800012 70.200012) (width 0.4) (layer B.Cu) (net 12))
 (segment (start 88.030001 76.820001) (end 92.486001 76.820001) (width 0.4) (layer B.Cu) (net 12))
 (segment (start 93.110001 74.080003) (end 92.049999 73.020001) (width 0.4) (layer B.Cu) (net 12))
 (segment (start 92.049999 70.779999) (end 92.629986 70.200012) (width 0.4) (layer B.Cu) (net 12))
 (segment (start 92.049999 73.020001) (end 92.049999 70.779999) (width 0.4) (layer B.Cu) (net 12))
 (segment (start 93.110001 76.196001) (end 93.110001 74.080003) (width 0.4) (layer B.Cu) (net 12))
 (segment (start 92.486001 76.820001) (end 93.110001 76.196001) (width 0.4) (layer B.Cu) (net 12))
 (segment (start 96.800012 70.200012) (end 97.9 71.3) (width 0.4) (layer B.Cu) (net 12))
 (segment (start 86.83 75.62) (end 88.030001 76.820001) (width 0.4) (layer B.Cu) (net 12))
 (segment (start 82.95 70.978608) (end 84.728608 70.978608) (width 0.4) (layer B.Cu) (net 13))
 (segment (start 84.728608 70.978608) (end 89.37 75.62) (width 0.4) (layer B.Cu) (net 13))
 (segment (start 83.496051 79.203949) (end 83.496051 83.749999) (width 0.4) (layer F.Cu) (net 13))
 (segment (start 83.496051 83.749999) (end 79.348025 87.898025) (width 0.4) (layer F.Cu) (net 13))
 (segment (start 89.37 75.62) (end 85.786051 79.203949) (width 0.4) (layer F.Cu) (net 13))
 (segment (start 85.786051 79.203949) (end 83.496051 79.203949) (width 0.4) (layer F.Cu) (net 13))
 (segment (start 103.8556 74.3242) (end 102.8758 74.3242) (width 0.4) (layer B.Cu) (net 14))
 (segment (start 102.8758 74.3242) (end 101.95 75.25) (width 0.4) (layer B.Cu) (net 14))
 (segment (start 102.088198 72.2668) (end 102.811802 72.2668) (width 0.4) (layer F.Cu) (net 14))
 (segment (start 102.811802 72.2668) (end 103.8556 73.310598) (width 0.4) (layer F.Cu) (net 14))
 (segment (start 103.8556 73.310598) (end 103.8556 74.3242) (width 0.4) (layer F.Cu) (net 14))
 (via (at 103.8556 74.3242) (size 0.6) (drill 0.4) (layers F.Cu B.Cu) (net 14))
 (segment (start 100.6806 74.864402) (end 100.6806 73.674398) (width 0.4) (layer F.Cu) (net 14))
 (segment (start 100.6806 73.674398) (end 102.088198 72.2668) (width 0.4) (layer F.Cu) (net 14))
 (segment (start 91.91 75.62) (end 93.110001 76.820001) (width 0.4) (layer F.Cu) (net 14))
 (segment (start 93.110001 76.820001) (end 98.725001 76.820001) (width 0.4) (layer F.Cu) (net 14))
 (segment (start 98.725001 76.820001) (end 100.6806 74.864402) (width 0.4) (layer F.Cu) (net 14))
 (segment (start 101.95 71.25) (end 101.95 72.65) (width 0.4) (layer B.Cu) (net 15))
 (segment (start 101.95 72.65) (end 100.515601 74.084399) (width 0.4) (layer B.Cu) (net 15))
 (segment (start 90.688199 105.561801) (end 89.85 106.4) (width 0.4) (layer B.Cu) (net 15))
 (segment (start 100.515601 74.084399) (end 100.515601 95.734399) (width 0.4) (layer B.Cu) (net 15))
 (segment (start 100.515601 95.734399) (end 90.688199 105.561801) (width 0.4) (layer B.Cu) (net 15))
 (segment (start 79.903949 79.203949) (end 78.665748 80.44215) (width 0.4) (layer F.Cu) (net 16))
 (segment (start 78.665748 80.44215) (end 78.665748 85.034252) (width 0.4) (layer F.Cu) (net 16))
 (segment (start 78.665748 85.034252) (end 77.389289 86.310711) (width 0.4) (layer F.Cu) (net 16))
 (segment (start 77.389289 86.310711) (end 77.365689 86.310711) (width 0.4) (layer F.Cu) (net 16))
 (segment (start 77.365689 86.310711) (end 76.8554 86.821) (width 0.4) (layer F.Cu) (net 16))
 (segment (start 76.8554 86.821) (end 76.8554 87.6554) (width 0.4) (layer F.Cu) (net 16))
 (segment (start 76.8554 87.6554) (end 78.597494 89.397494) (width 0.4) (layer F.Cu) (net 16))
 (segment (start 78.597494 89.397494) (end 79.644608 89.397494) (width 0.4) (layer F.Cu) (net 16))
 (segment (start 79.644608 89.397494) (end 80.246051 88.796051) (width 0.4) (layer F.Cu) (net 16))
 (segment (start 82.414838 108.433238) (end 82.414838 106.685162) (width 0.8) (layer B.Cu) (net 7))
 (segment (start 82.414838 106.685162) (end 83.371572 105.728428) (width 0.8) (layer B.Cu) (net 7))
 (segment (start 83.695 110) (end 83.695 109.7134) (width 0.8) (layer B.Cu) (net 7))
 (segment (start 83.695 109.7134) (end 82.414838 108.433238) (width 0.8) (layer B.Cu) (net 7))
 (segment (start 79.3954 105.49) (end 79.4716 105.49) (width 0.4) (layer B.Cu) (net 8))
 (segment (start 79.4716 105.49) (end 80.64 106.6584) (width 0.4) (layer B.Cu) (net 8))
 (segment (start 77.0586 101.5784) (end 77.0586 103.1532) (width 0.4) (layer F.Cu) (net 8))
 (segment (start 77.0586 103.1532) (end 79.3954 105.49) (width 0.4) (layer F.Cu) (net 8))
 (via (at 79.3954 105.49) (size 0.6) (drill 0.4) (layers F.Cu B.Cu) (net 8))
 (segment (start 77.846 100.791) (end 77.0586 101.5784) (width 0.4) (layer F.Cu) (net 8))
 (segment (start 77.846 98.006202) (end 77.846 100.791) (width 0.4) (layer F.Cu) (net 8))
 (segment (start 77.952201 97.900001) (end 77.846 98.006202) (width 0.4) (layer F.Cu) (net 8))
 (segment (start 77.2 97.75) (end 77.350001 97.900001) (width 0.4) (layer F.Cu) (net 8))
 (segment (start 77.350001 97.900001) (end 77.952201 97.900001) (width 0.4) (layer F.Cu) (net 8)))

